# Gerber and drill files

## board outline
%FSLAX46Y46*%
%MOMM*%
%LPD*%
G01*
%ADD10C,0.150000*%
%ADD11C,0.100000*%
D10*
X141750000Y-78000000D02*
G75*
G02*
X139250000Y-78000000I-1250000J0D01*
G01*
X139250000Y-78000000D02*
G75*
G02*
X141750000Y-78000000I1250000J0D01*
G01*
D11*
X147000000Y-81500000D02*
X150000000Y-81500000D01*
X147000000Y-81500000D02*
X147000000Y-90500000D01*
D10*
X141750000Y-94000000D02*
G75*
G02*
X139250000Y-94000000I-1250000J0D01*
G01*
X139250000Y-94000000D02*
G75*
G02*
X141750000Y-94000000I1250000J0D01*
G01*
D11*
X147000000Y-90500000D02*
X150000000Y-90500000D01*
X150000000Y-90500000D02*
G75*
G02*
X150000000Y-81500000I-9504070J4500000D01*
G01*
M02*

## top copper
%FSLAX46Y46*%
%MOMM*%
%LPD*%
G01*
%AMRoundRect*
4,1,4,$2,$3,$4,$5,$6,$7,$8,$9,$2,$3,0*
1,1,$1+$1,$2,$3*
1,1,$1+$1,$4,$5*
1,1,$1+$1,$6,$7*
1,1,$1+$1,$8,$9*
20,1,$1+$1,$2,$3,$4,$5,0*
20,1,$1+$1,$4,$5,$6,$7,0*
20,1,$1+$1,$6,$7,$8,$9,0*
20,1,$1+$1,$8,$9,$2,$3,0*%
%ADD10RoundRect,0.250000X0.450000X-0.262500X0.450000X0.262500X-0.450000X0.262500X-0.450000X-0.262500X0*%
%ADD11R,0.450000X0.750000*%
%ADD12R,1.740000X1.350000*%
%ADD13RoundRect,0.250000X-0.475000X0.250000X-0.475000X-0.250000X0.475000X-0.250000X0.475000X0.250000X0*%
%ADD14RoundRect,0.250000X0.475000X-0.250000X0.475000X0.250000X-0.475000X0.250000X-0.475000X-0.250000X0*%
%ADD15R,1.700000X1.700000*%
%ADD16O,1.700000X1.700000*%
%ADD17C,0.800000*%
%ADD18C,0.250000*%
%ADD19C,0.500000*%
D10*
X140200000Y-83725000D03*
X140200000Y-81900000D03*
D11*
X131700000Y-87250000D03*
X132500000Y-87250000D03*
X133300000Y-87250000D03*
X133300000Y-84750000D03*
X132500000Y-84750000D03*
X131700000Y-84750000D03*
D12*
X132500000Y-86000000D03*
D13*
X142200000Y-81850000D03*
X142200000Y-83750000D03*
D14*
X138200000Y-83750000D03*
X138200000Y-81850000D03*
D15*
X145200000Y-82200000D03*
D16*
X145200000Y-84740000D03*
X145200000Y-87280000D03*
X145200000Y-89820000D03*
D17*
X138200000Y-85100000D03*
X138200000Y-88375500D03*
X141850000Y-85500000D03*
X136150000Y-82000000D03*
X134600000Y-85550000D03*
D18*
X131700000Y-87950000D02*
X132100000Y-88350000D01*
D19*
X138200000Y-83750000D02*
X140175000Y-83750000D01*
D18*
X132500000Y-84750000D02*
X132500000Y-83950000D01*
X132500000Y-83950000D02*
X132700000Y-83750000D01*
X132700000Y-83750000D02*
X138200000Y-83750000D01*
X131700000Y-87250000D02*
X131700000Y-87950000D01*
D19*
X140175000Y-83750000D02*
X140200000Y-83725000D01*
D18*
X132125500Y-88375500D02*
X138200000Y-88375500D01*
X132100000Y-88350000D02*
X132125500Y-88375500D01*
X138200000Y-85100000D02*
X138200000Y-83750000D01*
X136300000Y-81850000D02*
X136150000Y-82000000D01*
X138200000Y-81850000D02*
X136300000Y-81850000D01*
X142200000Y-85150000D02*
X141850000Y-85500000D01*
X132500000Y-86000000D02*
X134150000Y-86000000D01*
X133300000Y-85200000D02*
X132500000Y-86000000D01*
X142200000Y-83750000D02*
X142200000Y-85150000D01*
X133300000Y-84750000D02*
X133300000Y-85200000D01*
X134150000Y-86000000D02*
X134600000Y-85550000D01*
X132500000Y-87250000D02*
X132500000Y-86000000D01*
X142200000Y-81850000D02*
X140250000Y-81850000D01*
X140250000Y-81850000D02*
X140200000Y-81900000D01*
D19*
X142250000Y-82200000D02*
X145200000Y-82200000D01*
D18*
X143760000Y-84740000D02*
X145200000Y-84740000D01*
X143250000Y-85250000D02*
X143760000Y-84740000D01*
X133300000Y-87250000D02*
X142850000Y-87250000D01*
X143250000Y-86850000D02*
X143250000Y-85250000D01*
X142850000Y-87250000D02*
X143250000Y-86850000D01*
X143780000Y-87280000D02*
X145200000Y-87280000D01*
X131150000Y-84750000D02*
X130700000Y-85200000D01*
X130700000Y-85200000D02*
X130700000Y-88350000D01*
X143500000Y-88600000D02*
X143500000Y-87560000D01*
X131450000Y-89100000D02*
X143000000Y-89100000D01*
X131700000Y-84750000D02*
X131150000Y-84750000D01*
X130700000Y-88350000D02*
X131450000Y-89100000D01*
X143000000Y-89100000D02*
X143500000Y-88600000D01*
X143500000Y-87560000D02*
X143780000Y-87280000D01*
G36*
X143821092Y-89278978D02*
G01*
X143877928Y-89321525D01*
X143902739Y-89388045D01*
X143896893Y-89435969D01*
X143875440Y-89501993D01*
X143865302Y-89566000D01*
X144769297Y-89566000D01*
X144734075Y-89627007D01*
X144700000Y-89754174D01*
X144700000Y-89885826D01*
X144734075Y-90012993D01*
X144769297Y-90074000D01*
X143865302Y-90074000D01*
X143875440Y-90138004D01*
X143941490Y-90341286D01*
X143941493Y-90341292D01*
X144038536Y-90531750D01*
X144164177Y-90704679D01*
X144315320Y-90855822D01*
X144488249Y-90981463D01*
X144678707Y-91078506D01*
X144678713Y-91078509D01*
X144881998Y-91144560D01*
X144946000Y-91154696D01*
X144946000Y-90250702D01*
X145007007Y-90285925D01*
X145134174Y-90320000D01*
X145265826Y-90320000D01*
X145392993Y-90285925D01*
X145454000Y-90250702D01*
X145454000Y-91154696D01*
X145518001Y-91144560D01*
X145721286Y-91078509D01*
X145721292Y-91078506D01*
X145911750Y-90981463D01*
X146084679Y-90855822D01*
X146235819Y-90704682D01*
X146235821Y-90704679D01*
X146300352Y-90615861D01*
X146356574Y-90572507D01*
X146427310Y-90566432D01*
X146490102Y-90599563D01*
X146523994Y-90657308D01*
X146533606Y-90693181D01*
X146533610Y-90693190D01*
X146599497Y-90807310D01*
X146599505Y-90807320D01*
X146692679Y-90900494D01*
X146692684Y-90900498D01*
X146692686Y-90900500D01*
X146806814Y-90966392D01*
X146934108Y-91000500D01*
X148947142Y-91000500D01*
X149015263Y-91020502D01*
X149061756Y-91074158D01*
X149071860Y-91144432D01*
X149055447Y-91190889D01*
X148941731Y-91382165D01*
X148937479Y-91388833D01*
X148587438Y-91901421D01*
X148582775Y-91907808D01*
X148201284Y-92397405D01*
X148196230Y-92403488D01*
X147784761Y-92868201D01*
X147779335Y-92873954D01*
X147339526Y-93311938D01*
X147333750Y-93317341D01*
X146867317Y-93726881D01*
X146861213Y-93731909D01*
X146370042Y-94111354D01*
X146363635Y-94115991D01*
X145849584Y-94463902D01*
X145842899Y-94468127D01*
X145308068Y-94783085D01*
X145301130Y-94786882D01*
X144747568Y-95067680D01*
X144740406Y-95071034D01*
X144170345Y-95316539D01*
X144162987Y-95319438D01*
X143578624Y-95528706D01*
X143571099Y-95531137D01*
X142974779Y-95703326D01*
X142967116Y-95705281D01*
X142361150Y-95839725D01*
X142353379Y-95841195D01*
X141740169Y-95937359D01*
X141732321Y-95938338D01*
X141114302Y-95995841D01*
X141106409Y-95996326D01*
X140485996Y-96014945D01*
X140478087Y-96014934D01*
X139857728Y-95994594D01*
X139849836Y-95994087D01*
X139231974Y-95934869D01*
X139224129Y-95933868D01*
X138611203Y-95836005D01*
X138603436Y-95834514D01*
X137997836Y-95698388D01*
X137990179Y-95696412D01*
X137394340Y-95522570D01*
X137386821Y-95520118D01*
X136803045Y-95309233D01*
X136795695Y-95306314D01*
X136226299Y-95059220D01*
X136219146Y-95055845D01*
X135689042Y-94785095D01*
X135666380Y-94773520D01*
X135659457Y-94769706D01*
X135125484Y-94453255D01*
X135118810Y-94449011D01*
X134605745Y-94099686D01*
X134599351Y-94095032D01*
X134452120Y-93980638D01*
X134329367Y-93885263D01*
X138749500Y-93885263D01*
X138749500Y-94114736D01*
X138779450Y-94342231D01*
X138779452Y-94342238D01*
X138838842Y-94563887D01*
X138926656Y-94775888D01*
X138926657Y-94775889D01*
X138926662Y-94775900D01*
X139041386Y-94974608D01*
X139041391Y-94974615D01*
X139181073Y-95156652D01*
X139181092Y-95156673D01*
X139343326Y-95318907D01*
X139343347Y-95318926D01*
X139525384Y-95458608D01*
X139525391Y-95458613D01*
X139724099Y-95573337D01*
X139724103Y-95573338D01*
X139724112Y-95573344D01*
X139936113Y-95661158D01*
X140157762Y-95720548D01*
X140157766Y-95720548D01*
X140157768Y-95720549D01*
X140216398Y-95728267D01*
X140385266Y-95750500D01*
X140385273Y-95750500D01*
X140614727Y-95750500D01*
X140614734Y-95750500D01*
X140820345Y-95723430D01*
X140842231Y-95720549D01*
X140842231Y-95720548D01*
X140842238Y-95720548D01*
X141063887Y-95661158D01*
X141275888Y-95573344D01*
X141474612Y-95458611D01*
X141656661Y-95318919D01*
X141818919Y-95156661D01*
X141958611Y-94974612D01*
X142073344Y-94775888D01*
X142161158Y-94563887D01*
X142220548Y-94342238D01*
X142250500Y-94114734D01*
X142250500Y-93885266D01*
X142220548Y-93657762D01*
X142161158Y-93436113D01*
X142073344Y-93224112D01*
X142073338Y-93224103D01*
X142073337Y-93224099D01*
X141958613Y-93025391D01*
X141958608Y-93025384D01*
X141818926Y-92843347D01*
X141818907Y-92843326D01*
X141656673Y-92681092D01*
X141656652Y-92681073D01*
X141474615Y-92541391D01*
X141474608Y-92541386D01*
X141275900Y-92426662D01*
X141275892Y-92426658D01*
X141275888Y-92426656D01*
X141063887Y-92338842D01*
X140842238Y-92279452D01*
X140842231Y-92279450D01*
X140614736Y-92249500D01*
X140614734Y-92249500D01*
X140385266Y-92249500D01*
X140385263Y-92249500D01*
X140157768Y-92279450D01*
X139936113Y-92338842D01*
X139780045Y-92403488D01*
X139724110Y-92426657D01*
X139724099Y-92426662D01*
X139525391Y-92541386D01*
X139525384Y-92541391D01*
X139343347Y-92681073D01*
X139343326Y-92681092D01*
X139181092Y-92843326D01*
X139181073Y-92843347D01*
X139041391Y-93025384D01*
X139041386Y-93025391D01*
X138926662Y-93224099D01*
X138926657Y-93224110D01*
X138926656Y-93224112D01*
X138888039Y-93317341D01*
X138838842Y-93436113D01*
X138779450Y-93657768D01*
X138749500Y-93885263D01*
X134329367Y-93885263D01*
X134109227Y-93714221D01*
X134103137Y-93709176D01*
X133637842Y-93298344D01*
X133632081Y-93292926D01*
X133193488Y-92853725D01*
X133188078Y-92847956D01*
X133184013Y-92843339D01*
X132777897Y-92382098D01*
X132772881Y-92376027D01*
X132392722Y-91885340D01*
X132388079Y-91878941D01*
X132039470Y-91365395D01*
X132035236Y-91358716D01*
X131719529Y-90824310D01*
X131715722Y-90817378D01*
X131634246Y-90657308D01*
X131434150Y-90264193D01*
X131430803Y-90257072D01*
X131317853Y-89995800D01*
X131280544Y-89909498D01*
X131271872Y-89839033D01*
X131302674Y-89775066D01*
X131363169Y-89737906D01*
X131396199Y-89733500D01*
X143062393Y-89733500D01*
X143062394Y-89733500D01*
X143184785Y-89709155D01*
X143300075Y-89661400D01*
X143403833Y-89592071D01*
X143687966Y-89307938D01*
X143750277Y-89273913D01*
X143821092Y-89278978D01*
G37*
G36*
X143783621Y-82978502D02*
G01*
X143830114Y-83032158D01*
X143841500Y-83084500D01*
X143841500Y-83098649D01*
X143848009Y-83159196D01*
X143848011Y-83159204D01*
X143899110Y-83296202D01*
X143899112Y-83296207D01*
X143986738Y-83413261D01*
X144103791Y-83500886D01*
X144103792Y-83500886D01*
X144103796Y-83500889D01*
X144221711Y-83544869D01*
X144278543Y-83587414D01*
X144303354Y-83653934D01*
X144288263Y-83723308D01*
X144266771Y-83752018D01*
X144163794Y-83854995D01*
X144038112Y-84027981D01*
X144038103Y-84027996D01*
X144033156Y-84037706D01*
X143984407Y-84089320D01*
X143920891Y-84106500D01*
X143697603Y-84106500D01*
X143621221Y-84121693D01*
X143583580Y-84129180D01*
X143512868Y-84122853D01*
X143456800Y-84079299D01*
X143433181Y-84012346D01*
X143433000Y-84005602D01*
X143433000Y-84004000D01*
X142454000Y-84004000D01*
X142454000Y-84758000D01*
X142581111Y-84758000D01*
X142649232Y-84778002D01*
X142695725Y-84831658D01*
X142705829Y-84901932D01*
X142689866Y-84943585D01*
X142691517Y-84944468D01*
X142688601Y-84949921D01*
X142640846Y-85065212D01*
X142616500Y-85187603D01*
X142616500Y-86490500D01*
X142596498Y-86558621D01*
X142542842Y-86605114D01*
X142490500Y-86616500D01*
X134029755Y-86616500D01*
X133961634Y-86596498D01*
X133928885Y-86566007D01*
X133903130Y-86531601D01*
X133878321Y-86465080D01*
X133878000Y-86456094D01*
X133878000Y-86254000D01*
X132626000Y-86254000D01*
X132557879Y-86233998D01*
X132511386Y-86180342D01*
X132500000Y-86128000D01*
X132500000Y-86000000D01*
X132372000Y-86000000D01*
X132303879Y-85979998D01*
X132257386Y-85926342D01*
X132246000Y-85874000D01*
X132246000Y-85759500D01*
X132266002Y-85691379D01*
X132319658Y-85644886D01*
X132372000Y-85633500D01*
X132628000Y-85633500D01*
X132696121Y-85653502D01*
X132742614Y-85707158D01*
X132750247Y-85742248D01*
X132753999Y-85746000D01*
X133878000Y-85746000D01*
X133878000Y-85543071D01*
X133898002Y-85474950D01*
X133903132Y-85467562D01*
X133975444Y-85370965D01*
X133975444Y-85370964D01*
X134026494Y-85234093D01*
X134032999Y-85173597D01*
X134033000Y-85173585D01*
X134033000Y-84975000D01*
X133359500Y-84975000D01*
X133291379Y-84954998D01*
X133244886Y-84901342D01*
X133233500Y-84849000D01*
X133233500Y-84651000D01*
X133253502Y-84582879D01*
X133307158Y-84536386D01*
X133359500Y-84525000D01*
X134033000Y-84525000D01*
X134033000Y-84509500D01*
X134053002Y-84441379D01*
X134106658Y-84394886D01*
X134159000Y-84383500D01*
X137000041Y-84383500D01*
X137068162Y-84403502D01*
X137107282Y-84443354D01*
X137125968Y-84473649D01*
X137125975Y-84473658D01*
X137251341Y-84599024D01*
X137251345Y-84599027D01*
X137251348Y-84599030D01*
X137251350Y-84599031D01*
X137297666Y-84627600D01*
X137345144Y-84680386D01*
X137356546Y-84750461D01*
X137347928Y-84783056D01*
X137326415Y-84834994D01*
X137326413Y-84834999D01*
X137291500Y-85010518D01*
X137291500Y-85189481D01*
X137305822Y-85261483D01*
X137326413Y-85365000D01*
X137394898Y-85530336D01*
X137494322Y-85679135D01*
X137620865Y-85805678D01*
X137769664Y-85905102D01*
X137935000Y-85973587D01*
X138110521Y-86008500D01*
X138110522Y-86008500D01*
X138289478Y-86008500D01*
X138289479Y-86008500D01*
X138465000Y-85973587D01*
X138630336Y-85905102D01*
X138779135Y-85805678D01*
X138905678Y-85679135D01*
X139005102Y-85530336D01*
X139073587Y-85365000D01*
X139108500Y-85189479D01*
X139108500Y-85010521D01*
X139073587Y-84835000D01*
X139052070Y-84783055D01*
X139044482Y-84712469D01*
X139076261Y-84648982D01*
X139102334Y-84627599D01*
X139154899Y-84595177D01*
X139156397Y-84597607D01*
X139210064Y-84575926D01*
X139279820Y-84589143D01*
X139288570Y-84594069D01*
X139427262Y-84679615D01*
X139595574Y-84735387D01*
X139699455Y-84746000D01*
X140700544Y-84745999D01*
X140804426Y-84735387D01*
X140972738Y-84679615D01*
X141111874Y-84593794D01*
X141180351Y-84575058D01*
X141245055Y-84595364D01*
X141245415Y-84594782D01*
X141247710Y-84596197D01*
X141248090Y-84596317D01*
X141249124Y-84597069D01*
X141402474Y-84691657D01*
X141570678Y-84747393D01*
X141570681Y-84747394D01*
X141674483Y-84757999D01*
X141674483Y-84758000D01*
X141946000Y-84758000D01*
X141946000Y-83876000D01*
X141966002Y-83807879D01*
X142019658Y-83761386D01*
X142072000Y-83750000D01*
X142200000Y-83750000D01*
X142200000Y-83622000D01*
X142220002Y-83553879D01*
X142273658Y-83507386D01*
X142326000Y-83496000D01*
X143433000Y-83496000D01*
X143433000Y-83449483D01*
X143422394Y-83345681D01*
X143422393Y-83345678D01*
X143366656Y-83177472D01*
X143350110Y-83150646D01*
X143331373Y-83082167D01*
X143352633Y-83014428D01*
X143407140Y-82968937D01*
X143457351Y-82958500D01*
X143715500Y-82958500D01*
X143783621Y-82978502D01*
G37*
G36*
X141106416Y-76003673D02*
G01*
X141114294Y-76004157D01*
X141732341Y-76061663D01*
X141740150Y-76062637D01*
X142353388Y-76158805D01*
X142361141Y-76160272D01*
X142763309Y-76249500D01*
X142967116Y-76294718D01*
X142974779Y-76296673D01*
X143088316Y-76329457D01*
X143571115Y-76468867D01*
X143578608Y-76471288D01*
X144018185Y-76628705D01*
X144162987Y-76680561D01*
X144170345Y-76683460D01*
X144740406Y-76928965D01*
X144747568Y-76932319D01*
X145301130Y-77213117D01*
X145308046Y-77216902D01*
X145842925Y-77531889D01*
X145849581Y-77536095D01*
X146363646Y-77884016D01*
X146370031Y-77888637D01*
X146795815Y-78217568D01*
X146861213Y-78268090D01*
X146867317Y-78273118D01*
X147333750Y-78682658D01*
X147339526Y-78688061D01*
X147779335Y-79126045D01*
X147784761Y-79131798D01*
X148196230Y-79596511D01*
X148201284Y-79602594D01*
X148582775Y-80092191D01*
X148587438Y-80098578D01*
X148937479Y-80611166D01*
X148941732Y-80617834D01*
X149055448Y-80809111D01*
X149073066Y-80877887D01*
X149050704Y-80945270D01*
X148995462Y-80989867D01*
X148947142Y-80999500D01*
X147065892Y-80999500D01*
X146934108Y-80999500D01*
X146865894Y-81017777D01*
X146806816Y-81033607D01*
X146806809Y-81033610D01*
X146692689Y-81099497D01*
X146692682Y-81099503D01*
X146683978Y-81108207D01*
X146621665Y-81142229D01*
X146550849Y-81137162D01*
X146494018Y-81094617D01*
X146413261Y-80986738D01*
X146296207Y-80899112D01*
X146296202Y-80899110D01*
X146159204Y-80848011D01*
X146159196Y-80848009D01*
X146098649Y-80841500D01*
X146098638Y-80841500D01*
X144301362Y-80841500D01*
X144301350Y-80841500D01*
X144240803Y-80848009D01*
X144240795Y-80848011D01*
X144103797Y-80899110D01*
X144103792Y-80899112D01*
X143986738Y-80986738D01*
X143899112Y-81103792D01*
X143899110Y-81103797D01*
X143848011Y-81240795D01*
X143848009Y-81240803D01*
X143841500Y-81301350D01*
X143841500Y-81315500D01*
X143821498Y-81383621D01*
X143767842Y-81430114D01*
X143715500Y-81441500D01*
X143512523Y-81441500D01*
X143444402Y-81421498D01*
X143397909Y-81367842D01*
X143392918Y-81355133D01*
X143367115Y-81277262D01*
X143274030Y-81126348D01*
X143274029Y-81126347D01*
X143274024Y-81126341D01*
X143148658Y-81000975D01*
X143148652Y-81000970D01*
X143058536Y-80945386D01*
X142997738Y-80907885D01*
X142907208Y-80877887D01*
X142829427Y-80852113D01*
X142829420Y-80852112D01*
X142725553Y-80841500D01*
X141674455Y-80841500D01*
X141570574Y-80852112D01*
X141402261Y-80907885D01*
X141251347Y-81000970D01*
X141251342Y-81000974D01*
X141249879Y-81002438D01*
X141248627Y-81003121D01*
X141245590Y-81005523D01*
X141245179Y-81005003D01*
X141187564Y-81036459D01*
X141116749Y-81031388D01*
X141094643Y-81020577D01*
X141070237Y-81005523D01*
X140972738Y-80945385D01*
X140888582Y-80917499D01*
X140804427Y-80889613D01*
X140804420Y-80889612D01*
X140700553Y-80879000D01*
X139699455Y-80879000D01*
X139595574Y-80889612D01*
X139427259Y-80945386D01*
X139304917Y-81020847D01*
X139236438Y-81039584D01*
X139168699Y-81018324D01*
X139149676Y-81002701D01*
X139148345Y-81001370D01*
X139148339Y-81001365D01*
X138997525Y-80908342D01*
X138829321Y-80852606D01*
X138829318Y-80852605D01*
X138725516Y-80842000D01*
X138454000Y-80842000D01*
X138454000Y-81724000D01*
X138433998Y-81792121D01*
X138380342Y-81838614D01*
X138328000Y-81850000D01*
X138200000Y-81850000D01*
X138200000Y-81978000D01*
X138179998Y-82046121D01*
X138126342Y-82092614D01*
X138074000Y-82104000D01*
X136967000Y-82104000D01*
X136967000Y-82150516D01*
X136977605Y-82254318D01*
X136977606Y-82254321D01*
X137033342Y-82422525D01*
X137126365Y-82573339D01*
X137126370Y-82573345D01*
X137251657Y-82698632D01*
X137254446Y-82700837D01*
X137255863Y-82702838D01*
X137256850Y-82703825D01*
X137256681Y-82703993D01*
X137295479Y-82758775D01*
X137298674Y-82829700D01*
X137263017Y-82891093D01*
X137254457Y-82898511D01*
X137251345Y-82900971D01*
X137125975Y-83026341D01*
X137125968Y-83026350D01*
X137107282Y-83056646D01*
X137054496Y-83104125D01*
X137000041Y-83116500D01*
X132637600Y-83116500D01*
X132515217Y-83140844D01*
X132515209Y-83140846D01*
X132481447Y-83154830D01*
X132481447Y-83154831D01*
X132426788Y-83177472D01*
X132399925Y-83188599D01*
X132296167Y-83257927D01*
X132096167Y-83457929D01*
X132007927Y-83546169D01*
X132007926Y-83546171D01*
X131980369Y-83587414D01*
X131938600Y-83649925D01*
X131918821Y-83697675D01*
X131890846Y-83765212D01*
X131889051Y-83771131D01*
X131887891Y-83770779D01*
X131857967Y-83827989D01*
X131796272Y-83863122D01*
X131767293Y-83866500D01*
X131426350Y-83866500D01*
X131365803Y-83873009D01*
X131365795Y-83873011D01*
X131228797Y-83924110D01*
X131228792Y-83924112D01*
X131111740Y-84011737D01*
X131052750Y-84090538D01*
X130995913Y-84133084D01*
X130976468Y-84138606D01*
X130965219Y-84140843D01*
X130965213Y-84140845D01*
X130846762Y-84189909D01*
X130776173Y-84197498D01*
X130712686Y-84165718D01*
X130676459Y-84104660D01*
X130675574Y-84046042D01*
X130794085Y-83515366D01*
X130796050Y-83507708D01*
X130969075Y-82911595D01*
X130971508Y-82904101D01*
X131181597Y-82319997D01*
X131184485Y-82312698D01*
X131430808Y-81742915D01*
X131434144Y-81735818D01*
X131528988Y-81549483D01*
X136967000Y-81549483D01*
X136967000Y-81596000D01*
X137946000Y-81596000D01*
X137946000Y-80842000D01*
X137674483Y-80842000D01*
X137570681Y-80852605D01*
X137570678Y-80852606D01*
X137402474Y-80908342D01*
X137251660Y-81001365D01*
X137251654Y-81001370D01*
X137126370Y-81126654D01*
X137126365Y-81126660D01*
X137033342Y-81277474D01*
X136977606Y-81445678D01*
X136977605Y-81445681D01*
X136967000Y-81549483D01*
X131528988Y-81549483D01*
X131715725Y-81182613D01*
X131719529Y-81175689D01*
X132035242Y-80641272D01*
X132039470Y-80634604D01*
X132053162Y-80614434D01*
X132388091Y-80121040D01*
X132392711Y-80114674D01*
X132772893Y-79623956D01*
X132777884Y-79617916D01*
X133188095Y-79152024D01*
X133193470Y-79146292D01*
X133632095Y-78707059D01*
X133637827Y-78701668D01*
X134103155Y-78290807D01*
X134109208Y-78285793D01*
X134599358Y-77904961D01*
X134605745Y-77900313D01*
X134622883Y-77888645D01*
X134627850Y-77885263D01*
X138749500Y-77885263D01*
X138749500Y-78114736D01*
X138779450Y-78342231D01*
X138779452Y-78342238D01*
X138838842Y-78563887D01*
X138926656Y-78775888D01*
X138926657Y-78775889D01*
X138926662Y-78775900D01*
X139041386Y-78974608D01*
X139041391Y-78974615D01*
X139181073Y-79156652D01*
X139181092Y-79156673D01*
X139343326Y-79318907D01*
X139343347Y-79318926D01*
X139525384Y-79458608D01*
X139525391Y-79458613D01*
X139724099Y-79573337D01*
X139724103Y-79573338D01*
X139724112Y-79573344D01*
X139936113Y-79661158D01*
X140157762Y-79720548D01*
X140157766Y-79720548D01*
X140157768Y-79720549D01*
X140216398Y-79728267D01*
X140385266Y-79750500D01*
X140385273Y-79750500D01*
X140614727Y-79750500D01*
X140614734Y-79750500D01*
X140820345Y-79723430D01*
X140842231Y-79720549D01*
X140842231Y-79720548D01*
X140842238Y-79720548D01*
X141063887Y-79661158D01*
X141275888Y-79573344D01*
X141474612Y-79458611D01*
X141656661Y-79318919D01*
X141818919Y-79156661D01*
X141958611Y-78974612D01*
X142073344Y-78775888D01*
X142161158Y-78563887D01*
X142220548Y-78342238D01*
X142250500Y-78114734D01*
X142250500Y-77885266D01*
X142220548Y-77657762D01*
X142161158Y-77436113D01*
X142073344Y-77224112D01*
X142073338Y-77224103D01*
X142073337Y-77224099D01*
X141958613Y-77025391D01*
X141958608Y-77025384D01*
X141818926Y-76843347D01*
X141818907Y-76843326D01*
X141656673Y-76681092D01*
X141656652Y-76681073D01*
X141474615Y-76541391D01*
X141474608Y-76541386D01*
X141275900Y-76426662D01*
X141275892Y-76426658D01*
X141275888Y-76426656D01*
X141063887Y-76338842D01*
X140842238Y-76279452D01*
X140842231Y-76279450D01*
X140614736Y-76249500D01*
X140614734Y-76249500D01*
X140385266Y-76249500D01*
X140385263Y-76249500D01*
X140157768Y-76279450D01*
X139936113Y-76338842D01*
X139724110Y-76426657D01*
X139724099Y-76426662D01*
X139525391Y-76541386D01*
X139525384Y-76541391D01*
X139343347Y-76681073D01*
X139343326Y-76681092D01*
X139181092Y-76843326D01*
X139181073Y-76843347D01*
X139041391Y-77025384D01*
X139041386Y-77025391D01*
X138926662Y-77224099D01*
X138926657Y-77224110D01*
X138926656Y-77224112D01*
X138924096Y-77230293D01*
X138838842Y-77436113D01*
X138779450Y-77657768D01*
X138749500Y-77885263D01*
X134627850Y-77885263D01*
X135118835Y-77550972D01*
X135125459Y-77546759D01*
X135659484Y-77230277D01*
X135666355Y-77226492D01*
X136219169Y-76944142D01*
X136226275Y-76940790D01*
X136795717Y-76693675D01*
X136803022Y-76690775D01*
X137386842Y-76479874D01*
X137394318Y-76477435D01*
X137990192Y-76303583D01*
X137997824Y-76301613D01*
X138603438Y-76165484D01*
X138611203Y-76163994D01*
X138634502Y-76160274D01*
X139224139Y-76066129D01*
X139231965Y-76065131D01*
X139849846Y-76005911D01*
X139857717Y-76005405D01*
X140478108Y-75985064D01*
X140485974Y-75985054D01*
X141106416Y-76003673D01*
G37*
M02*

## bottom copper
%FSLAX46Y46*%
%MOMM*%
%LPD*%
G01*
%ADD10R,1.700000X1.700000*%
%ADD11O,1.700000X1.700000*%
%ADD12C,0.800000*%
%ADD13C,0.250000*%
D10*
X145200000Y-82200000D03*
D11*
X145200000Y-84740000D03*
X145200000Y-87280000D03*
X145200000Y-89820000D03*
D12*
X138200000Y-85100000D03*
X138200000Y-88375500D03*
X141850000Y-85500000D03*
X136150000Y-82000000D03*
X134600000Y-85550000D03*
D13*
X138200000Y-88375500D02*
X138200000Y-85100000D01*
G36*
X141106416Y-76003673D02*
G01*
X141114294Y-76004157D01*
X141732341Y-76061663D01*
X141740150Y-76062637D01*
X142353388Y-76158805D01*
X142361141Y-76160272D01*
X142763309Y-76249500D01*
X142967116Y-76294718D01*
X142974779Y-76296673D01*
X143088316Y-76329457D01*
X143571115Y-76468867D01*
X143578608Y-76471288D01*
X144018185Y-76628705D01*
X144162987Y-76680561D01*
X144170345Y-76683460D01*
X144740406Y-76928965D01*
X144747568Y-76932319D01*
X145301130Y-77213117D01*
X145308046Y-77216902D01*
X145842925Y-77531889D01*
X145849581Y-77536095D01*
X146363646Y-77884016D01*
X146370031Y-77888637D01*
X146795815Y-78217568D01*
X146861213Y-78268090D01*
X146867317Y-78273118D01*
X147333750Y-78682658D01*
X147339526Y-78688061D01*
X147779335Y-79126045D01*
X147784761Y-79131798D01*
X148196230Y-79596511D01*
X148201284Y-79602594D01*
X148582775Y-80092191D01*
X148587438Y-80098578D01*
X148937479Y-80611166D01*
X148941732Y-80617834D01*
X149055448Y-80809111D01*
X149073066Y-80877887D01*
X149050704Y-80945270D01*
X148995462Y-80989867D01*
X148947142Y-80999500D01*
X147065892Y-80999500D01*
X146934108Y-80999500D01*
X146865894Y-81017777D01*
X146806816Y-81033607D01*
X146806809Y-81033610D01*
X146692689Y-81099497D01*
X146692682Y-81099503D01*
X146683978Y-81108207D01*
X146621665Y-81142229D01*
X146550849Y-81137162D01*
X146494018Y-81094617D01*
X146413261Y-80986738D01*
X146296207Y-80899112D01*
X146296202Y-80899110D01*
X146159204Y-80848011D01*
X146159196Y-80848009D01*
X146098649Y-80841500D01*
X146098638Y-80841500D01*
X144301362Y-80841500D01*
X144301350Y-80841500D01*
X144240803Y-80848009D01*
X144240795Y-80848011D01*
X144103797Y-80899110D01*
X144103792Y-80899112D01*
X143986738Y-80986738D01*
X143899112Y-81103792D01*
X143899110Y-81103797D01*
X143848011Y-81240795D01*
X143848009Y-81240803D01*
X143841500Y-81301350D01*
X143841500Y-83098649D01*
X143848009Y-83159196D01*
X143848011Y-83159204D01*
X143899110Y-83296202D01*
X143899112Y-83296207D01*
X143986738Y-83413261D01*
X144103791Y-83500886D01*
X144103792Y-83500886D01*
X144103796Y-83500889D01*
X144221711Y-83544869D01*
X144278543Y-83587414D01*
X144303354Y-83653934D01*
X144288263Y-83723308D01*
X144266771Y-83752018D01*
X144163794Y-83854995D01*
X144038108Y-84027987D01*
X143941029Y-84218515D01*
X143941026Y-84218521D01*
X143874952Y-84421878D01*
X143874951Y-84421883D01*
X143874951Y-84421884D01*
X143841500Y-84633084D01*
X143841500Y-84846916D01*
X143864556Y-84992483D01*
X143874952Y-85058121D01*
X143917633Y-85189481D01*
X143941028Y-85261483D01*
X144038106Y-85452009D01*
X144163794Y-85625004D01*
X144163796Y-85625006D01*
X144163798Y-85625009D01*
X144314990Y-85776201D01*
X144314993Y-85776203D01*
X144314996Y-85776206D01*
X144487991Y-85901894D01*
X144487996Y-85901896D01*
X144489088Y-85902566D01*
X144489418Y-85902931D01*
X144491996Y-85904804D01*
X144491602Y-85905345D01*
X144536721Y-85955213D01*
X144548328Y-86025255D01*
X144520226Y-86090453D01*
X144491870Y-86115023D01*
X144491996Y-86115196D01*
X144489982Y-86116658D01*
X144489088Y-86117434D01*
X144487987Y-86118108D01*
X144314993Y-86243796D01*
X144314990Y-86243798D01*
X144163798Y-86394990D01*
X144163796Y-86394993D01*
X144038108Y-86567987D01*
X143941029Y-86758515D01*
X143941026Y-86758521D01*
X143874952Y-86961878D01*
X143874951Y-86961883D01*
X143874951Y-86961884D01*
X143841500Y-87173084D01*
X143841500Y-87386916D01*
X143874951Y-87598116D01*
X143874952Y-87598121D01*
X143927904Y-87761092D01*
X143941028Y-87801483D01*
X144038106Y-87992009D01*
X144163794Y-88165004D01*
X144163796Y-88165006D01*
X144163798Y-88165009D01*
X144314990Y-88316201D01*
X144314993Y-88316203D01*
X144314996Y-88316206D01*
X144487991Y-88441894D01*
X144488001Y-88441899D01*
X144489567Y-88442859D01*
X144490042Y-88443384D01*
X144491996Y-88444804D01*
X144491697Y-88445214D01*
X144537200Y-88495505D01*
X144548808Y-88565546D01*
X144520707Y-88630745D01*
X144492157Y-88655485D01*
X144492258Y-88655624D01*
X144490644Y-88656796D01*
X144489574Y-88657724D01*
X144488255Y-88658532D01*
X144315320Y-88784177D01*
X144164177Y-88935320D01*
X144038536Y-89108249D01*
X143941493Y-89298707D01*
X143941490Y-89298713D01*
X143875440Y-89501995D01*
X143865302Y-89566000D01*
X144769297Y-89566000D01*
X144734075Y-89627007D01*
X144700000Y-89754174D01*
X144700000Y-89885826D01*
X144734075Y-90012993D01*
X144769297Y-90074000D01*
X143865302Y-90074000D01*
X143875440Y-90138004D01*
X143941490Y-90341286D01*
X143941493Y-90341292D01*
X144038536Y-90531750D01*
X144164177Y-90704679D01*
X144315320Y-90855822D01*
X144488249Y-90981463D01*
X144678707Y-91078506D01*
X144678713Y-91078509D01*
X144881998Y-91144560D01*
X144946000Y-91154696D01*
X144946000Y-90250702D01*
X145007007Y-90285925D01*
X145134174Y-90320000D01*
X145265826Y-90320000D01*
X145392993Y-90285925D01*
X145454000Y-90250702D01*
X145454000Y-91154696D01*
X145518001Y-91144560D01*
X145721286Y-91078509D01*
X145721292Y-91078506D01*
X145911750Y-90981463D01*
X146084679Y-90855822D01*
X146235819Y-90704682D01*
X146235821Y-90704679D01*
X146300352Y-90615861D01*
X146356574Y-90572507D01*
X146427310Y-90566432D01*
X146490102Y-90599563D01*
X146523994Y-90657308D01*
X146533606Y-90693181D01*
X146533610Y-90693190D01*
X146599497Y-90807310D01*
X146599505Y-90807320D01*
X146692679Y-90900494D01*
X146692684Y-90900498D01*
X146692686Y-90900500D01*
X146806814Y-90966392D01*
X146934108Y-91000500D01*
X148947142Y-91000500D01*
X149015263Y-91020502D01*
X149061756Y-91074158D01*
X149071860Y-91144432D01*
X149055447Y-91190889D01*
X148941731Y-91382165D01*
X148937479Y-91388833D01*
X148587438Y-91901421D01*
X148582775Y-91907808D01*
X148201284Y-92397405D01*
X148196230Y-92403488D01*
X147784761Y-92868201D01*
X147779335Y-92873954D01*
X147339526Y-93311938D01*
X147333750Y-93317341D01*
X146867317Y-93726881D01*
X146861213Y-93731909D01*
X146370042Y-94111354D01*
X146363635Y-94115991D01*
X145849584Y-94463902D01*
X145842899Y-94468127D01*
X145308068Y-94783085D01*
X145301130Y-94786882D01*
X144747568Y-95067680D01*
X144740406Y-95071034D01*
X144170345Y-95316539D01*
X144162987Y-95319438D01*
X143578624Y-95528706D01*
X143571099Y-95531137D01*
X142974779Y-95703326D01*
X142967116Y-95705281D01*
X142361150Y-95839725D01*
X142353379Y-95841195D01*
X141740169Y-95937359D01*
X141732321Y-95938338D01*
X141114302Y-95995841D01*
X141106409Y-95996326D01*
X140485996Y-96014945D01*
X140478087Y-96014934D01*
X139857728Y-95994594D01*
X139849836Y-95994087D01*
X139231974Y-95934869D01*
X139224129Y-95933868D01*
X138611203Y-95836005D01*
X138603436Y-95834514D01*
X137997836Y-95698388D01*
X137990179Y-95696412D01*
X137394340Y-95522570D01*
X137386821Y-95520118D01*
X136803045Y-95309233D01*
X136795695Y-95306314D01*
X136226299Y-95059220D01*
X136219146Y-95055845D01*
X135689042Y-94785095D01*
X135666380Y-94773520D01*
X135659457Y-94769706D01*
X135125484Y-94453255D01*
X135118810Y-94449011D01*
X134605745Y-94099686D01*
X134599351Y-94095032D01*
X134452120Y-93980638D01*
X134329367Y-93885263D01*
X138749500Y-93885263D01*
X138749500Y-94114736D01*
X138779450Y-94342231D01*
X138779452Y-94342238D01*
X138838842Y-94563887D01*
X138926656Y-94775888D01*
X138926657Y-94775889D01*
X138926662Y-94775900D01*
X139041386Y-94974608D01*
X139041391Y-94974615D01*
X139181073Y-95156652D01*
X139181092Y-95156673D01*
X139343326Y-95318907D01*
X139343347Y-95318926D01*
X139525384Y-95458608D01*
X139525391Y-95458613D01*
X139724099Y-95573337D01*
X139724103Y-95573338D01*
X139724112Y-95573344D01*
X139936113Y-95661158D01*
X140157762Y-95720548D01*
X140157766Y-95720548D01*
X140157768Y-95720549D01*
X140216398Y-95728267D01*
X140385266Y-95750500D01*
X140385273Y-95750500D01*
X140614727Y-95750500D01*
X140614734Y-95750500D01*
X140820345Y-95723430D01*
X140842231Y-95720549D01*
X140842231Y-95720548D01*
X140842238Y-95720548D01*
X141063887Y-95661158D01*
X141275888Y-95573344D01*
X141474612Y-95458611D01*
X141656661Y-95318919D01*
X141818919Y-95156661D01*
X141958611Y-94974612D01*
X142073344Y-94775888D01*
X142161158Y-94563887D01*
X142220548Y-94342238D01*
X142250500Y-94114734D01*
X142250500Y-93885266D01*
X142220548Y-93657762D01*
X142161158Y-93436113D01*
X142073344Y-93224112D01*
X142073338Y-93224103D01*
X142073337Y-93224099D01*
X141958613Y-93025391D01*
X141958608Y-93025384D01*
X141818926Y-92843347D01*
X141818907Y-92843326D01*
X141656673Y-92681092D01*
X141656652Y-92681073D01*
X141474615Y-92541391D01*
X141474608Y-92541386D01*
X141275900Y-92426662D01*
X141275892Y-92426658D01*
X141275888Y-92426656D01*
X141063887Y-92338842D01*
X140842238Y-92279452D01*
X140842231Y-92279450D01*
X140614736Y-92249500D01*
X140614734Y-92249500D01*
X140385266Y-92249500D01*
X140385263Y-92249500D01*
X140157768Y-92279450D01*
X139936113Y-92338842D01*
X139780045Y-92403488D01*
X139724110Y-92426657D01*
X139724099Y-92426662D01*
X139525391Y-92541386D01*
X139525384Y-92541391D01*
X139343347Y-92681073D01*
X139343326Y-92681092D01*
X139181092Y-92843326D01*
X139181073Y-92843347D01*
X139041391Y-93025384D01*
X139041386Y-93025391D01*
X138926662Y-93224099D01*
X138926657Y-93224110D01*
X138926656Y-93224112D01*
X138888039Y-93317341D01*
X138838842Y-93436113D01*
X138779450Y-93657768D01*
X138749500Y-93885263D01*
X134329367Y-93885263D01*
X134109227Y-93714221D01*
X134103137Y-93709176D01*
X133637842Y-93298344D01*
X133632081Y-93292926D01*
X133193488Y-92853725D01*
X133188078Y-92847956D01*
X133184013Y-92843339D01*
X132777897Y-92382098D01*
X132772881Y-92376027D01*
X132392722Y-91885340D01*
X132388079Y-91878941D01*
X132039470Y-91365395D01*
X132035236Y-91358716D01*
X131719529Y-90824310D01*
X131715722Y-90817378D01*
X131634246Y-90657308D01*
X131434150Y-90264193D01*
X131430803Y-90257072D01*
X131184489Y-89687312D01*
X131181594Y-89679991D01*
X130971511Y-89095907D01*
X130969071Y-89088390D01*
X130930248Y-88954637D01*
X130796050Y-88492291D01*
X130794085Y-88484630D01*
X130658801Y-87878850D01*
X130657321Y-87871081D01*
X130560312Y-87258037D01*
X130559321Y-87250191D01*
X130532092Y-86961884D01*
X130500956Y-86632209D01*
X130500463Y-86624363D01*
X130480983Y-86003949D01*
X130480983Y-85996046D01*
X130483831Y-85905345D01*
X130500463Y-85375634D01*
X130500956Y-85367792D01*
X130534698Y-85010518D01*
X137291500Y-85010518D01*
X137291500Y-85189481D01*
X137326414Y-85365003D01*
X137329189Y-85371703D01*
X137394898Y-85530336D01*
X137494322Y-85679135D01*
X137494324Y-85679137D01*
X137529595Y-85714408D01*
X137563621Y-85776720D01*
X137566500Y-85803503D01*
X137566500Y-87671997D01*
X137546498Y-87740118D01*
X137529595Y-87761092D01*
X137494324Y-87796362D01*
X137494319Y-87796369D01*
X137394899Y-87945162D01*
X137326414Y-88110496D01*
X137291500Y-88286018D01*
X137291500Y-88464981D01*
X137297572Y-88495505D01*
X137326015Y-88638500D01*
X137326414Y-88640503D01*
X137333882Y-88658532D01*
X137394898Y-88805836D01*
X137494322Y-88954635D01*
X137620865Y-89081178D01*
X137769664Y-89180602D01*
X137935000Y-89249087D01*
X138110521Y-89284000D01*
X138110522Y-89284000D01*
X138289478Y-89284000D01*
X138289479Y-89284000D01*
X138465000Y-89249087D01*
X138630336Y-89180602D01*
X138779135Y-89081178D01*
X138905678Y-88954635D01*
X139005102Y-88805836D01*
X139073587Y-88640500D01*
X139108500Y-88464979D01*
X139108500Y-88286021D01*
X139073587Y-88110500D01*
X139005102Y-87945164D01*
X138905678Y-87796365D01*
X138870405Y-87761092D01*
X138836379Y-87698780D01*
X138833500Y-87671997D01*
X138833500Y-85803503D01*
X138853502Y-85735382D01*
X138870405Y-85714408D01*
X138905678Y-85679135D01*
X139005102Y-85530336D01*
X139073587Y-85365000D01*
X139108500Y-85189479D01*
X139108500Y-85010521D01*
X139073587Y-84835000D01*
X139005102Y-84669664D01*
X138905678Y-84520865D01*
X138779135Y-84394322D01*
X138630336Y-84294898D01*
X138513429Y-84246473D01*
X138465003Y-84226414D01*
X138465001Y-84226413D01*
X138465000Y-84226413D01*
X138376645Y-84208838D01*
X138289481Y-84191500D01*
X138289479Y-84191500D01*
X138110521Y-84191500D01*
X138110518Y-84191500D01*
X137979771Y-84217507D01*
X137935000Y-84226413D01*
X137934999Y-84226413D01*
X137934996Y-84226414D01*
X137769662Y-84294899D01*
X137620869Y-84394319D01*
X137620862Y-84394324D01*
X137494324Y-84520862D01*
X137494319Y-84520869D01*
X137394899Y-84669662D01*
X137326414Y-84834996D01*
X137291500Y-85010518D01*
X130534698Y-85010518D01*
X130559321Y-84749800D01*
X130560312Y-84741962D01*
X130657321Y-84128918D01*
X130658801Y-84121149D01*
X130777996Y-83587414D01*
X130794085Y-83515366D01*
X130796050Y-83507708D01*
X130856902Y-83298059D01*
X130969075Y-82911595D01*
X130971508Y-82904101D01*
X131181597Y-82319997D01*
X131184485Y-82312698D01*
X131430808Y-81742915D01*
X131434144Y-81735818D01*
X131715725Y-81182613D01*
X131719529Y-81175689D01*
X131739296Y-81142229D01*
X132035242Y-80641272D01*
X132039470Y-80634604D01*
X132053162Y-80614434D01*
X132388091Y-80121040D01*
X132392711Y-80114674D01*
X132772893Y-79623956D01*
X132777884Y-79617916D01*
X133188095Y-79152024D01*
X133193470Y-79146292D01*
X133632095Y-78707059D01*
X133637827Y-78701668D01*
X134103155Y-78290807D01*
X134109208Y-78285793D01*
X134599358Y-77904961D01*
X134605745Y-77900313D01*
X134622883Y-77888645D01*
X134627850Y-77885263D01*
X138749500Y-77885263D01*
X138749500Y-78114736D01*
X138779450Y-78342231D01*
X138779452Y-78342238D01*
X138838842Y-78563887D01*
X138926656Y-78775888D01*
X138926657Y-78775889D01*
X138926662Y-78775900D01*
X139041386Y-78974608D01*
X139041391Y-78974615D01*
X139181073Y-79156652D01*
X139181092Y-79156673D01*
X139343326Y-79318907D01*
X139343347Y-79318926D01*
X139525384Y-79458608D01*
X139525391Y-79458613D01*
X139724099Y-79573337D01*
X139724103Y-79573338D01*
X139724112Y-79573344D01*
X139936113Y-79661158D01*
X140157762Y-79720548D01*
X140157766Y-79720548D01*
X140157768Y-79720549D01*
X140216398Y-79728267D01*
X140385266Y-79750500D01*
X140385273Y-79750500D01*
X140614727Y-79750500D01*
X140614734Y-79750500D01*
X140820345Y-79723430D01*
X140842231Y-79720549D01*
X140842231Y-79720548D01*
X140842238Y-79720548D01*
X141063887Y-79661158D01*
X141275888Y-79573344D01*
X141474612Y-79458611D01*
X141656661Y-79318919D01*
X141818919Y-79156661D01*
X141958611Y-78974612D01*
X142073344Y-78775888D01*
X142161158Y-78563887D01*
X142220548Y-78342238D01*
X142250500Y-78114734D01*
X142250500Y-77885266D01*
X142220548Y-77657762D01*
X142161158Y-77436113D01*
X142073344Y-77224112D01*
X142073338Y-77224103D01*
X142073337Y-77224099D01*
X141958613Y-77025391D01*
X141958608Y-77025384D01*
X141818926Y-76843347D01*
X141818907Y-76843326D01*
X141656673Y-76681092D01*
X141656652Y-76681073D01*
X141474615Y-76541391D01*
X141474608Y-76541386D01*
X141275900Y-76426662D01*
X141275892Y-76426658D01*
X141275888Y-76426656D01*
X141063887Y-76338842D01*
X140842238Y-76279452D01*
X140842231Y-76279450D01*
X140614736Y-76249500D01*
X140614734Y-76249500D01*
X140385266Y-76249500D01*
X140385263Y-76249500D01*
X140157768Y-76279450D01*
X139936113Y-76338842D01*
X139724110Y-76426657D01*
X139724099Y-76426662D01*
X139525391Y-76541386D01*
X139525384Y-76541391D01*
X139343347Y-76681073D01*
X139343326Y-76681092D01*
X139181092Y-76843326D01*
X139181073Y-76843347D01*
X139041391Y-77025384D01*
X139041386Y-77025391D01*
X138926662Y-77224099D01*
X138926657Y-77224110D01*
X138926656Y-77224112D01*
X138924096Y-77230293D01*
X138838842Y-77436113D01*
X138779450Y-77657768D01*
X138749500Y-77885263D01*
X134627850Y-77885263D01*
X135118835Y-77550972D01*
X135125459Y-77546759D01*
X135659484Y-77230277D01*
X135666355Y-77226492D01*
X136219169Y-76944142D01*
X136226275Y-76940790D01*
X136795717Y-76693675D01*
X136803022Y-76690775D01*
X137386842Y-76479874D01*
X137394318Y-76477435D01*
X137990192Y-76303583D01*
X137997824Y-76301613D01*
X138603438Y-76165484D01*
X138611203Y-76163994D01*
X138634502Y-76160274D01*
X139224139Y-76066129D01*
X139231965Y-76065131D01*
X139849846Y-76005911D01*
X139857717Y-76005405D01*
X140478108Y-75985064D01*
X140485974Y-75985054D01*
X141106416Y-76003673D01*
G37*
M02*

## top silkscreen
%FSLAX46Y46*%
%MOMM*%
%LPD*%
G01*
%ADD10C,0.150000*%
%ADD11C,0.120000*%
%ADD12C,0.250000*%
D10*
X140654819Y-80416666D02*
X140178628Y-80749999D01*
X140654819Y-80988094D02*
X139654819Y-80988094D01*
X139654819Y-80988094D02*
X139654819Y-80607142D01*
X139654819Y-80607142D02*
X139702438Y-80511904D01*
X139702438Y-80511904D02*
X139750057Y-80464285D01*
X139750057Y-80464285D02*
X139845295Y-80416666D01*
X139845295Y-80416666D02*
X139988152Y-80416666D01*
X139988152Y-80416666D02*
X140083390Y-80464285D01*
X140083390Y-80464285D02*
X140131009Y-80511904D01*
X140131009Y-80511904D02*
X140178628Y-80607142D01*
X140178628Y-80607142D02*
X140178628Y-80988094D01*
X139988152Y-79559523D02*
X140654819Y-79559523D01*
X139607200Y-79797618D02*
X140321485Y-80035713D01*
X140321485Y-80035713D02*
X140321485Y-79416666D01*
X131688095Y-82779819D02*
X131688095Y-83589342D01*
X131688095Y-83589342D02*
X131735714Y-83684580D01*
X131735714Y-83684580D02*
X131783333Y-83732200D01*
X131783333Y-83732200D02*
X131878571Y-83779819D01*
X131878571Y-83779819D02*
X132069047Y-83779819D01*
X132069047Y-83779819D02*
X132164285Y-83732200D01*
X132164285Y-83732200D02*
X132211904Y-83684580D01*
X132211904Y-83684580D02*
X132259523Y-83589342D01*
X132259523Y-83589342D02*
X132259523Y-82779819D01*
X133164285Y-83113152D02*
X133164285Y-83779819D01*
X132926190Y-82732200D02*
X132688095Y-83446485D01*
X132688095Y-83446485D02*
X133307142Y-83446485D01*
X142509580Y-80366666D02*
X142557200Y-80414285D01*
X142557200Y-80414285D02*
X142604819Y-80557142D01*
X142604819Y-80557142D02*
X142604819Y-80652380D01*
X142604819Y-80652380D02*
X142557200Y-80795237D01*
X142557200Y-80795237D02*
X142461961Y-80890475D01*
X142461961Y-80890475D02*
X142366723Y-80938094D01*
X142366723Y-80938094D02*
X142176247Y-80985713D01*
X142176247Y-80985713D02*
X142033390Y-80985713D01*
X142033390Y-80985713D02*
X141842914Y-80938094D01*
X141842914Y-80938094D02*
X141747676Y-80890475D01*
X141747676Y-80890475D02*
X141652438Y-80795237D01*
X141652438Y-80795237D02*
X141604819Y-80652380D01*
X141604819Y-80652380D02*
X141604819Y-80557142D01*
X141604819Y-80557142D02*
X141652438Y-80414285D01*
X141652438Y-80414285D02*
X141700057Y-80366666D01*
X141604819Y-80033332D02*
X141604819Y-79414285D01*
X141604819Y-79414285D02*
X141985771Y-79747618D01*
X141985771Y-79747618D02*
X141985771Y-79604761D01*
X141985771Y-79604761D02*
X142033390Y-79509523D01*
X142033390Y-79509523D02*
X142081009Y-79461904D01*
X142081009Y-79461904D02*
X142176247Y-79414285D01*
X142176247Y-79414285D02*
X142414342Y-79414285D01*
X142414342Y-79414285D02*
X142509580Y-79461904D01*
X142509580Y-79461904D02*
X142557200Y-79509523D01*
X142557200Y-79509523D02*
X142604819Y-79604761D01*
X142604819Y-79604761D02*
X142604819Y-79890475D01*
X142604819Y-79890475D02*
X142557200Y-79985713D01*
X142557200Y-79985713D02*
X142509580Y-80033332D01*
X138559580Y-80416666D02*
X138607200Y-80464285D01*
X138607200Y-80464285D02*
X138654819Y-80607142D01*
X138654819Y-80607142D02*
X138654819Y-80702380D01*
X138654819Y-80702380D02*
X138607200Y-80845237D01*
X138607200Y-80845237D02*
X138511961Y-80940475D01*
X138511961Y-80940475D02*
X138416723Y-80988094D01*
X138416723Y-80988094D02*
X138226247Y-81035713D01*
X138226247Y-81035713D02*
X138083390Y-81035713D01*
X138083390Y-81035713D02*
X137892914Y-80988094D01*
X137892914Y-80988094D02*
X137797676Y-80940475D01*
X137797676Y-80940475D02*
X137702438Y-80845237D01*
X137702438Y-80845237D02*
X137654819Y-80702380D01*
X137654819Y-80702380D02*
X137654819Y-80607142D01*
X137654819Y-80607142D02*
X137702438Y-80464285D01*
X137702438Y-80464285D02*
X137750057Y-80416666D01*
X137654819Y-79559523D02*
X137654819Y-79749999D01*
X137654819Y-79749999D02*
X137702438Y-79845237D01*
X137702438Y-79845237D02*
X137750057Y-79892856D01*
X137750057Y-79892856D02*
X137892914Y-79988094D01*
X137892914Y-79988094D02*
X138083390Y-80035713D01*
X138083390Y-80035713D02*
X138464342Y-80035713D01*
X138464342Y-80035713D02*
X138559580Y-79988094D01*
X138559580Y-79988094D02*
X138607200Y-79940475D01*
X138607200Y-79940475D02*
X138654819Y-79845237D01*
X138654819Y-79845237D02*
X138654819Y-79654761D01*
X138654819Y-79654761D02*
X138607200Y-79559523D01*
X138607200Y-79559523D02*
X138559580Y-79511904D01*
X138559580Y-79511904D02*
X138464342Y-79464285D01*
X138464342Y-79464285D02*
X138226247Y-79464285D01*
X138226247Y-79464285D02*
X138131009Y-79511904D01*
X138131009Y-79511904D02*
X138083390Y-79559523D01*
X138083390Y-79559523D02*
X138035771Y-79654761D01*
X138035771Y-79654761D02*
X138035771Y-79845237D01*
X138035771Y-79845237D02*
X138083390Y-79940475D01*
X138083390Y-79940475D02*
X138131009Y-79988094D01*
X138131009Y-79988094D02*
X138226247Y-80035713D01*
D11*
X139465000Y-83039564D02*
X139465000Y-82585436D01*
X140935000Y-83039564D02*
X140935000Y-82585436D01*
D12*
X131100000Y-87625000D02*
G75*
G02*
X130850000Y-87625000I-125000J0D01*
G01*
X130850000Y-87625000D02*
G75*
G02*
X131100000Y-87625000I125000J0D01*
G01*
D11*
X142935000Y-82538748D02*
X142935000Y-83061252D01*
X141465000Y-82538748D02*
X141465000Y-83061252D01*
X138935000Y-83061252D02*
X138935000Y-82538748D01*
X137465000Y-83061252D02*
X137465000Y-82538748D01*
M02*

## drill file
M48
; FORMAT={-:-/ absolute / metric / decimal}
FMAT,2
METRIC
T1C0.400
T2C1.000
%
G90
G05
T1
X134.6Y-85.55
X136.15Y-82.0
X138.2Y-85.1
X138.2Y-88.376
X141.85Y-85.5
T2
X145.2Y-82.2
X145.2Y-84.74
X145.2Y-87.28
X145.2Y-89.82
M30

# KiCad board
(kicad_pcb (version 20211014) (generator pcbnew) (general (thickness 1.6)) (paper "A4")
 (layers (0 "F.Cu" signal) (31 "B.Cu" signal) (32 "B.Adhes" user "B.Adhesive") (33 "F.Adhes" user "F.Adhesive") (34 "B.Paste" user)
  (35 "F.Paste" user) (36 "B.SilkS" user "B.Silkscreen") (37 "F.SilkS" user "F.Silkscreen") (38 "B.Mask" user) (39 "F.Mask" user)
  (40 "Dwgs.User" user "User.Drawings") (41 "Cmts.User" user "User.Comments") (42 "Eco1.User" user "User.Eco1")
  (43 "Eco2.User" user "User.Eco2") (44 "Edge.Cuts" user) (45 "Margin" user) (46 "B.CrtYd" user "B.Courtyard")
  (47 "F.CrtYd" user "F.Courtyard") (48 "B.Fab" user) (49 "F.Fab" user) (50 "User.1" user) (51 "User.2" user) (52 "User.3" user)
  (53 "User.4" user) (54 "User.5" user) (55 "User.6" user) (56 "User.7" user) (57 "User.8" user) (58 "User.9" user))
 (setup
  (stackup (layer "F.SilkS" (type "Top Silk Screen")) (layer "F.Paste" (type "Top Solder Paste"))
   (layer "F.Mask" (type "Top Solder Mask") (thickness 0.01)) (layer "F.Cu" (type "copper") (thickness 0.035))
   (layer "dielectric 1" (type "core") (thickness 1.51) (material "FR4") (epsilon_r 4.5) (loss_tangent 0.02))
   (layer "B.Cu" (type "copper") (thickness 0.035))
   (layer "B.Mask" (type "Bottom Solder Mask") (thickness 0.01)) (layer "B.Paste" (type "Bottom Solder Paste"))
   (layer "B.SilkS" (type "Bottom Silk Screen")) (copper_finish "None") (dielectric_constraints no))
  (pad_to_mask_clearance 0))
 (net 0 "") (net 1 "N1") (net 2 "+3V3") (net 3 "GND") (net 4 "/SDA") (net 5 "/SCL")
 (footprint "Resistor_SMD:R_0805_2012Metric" (layer "F.Cu") (at 140.2 82.8125 90)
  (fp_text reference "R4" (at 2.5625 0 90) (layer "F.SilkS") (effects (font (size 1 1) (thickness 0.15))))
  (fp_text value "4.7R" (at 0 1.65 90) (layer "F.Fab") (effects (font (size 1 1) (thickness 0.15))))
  (fp_line (start -0.227064 -0.735) (end 0.227064 -0.735) (layer "F.SilkS") (width 0.12))
  (fp_line (start -0.227064 0.735) (end 0.227064 0.735) (layer "F.SilkS") (width 0.12))
  (pad "1" smd roundrect locked (at -0.9125 0 90) (size 1.025 1.4) (layers "F.Cu" "F.Paste" "F.Mask") (roundrect_rratio 0.243902439)
   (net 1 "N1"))
  (pad "2" smd roundrect locked (at 0.9125 0 90) (size 1.025 1.4) (layers "F.Cu" "F.Paste" "F.Mask") (roundrect_rratio 0.243902439)
   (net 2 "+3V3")))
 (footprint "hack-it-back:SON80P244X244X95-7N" (layer "F.Cu") (at 132.5 86 90)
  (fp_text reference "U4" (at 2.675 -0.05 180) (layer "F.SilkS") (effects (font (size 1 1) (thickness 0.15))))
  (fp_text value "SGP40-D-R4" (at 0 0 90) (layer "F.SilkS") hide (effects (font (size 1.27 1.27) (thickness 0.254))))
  (fp_circle (center -1.625 -1.525) (end -1.625 -1.4) (layer "F.SilkS") (width 0.25) (fill none))
  (pad "1" smd rect (at -1.25 -0.8 180) (size 0.45 0.75) (layers "F.Cu" "F.Paste" "F.Mask") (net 1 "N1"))
  (pad "2" smd rect (at -1.25 0 180) (size 0.45 0.75) (layers "F.Cu" "F.Paste" "F.Mask") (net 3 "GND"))
  (pad "3" smd rect (at -1.25 0.8 180) (size 0.45 0.75) (layers "F.Cu" "F.Paste" "F.Mask") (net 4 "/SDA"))
  (pad "4" smd rect (at 1.25 0.8 180) (size 0.45 0.75) (layers "F.Cu" "F.Paste" "F.Mask") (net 3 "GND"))
  (pad "5" smd rect (at 1.25 0 180) (size 0.45 0.75) (layers "F.Cu" "F.Paste" "F.Mask") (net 1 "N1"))
  (pad "6" smd rect (at 1.25 -0.8 180) (size 0.45 0.75) (layers "F.Cu" "F.Paste" "F.Mask") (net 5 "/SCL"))
  (pad "7" smd rect (at 0 0 90) (size 1.35 1.74) (layers "F.Cu" "F.Paste" "F.Mask") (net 3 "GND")))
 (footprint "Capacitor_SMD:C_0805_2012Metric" (layer "F.Cu") (at 142.2 82.8 -90)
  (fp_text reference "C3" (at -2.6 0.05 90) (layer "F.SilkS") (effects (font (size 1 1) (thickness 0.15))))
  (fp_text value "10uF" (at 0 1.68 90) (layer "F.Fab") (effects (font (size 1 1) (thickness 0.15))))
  (fp_line (start -0.261252 -0.735) (end 0.261252 -0.735) (layer "F.SilkS") (width 0.12))
  (fp_line (start -0.261252 0.735) (end 0.261252 0.735) (layer "F.SilkS") (width 0.12))
  (pad "1" smd roundrect locked (at -0.95 0 270) (size 1 1.45) (layers "F.Cu" "F.Paste" "F.Mask") (roundrect_rratio 0.25) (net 2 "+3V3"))
  (pad "2" smd roundrect locked (at 0.95 0 270) (size 1 1.45) (layers "F.Cu" "F.Paste" "F.Mask") (roundrect_rratio 0.25) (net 3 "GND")))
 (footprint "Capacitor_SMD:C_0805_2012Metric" (layer "F.Cu") (at 138.2 82.8 90)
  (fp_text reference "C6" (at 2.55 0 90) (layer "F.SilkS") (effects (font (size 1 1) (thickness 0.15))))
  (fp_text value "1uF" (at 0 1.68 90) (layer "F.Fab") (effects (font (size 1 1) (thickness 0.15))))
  (fp_line (start -0.261252 0.735) (end 0.261252 0.735) (layer "F.SilkS") (width 0.12))
  (fp_line (start -0.261252 -0.735) (end 0.261252 -0.735) (layer "F.SilkS") (width 0.12))
  (pad "1" smd roundrect locked (at -0.95 0 90) (size 1 1.45) (layers "F.Cu" "F.Paste" "F.Mask") (roundrect_rratio 0.25) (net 1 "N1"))
  (pad "2" smd roundrect locked (at 0.95 0 90) (size 1 1.45) (layers "F.Cu" "F.Paste" "F.Mask") (roundrect_rratio 0.25) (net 3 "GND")))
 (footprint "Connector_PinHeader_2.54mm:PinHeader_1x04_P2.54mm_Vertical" (layer "B.Cu") (at 145.2 82.2 180)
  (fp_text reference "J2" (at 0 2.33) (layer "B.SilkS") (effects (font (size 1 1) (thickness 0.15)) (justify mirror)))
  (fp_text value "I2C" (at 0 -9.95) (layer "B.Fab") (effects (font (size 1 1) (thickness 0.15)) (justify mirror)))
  (pad "1" thru_hole rect locked (at 0 0 180) (size 1.7 1.7) (drill 1) (layers *.Cu *.Mask) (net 2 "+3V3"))
  (pad "2" thru_hole oval locked (at 0 -2.54 180) (size 1.7 1.7) (drill 1) (layers *.Cu *.Mask) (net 4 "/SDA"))
  (pad "3" thru_hole oval locked (at 0 -5.08 180) (size 1.7 1.7) (drill 1) (layers *.Cu *.Mask) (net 5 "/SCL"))
  (pad "4" thru_hole oval locked (at 0 -7.62 180) (size 1.7 1.7) (drill 1) (layers *.Cu *.Mask) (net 3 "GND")))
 (gr_circle (center 140.5 78) (end 141.75 78) (layer "Edge.Cuts") (width 0.15) (fill none))
 (gr_line (start 147 81.5) (end 150 81.5) (layer "Edge.Cuts") (width 0.1))
 (gr_line (start 147 81.5) (end 147 90.5) (layer "Edge.Cuts") (width 0.1))
 (gr_circle (center 140.5 94) (end 141.75 94) (layer "Edge.Cuts") (width 0.15) (fill none))
 (gr_line (start 147 90.5) (end 150 90.5) (layer "Edge.Cuts") (width 0.1))
 (gr_arc (start 150 90.5) (mid 129.980359 86) (end 150 81.5) (layer "Edge.Cuts") (width 0.1))
 (segment (start 131.7 87.95) (end 132.1 88.35) (width 0.25) (layer "F.Cu") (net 1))
 (segment (start 138.2 83.75) (end 140.175 83.75) (width 0.5) (layer "F.Cu") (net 1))
 (segment (start 132.5 84.75) (end 132.5 83.95) (width 0.25) (layer "F.Cu") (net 1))
 (segment (start 132.5 83.95) (end 132.7 83.75) (width 0.25) (layer "F.Cu") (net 1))
 (segment (start 132.7 83.75) (end 138.2 83.75) (width 0.25) (layer "F.Cu") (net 1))
 (segment (start 131.7 87.25) (end 131.7 87.95) (width 0.25) (layer "F.Cu") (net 1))
 (segment (start 140.175 83.75) (end 140.2 83.725) (width 0.5) (layer "F.Cu") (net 1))
 (segment (start 132.1255 88.3755) (end 138.2 88.3755) (width 0.25) (layer "F.Cu") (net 1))
 (segment (start 132.1 88.35) (end 132.1255 88.3755) (width 0.25) (layer "F.Cu") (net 1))
 (segment (start 138.2 85.1) (end 138.2 83.75) (width 0.25) (layer "F.Cu") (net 1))
 (via (at 138.2 85.1) (size 0.8) (drill 0.4) (layers "F.Cu" "B.Cu") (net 1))
 (via (at 138.2 88.3755) (size 0.8) (drill 0.4) (layers "F.Cu" "B.Cu") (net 1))
 (segment (start 138.2 88.3755) (end 138.2 85.1) (width 0.25) (layer "B.Cu") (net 1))
 (segment (start 136.3 81.85) (end 136.15 82) (width 0.25) (layer "F.Cu") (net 3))
 (segment (start 138.2 81.85) (end 136.3 81.85) (width 0.25) (layer "F.Cu") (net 3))
 (segment (start 142.2 85.15) (end 141.85 85.5) (width 0.25) (layer "F.Cu") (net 3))
 (segment (start 132.5 86) (end 134.15 86) (width 0.25) (layer "F.Cu") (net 3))
 (segment (start 133.3 85.2) (end 132.5 86) (width 0.25) (layer "F.Cu") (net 3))
 (segment (start 142.2 83.75) (end 142.2 85.15) (width 0.25) (layer "F.Cu") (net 3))
 (segment (start 133.3 84.75) (end 133.3 85.2) (width 0.25) (layer "F.Cu") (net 3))
 (segment (start 134.15 86) (end 134.6 85.55) (width 0.25) (layer "F.Cu") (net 3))
 (segment (start 132.5 87.25) (end 132.5 86) (width 0.25) (layer "F.Cu") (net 3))
 (via (at 141.85 85.5) (size 0.8) (drill 0.4) (layers "F.Cu" "B.Cu") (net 3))
 (via (at 136.15 82) (size 0.8) (drill 0.4) (layers "F.Cu" "B.Cu") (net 3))
 (via (at 134.6 85.55) (size 0.8) (drill 0.4) (layers "F.Cu" "B.Cu") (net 3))
 (segment (start 142.2 81.85) (end 140.25 81.85) (width 0.25) (layer "F.Cu") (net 2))
 (segment (start 140.25 81.85) (end 140.2 81.9) (width 0.25) (layer "F.Cu") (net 2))
 (segment (start 142.25 82.2) (end 145.2 82.2) (width 0.5) (layer "F.Cu") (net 2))
 (segment (start 143.76 84.74) (end 145.2 84.74) (width 0.25) (layer "F.Cu") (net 4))
 (segment (start 143.25 85.25) (end 143.76 84.74) (width 0.25) (layer "F.Cu") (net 4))
 (segment (start 133.3 87.25) (end 142.85 87.25) (width 0.25) (layer "F.Cu") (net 4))
 (segment (start 143.25 86.85) (end 143.25 85.25) (width 0.25) (layer "F.Cu") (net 4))
 (segment (start 142.85 87.25) (end 143.25 86.85) (width 0.25) (layer "F.Cu") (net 4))
 (segment (start 143.78 87.28) (end 145.2 87.28) (width 0.25) (layer "F.Cu") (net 5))
 (segment (start 131.15 84.75) (end 130.7 85.2) (width 0.25) (layer "F.Cu") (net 5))
 (segment (start 130.7 85.2) (end 130.7 88.35) (width 0.25) (layer "F.Cu") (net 5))
 (segment (start 143.5 88.6) (end 143.5 87.56) (width 0.25) (layer "F.Cu") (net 5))
 (segment (start 131.45 89.1) (end 143 89.1) (width 0.25) (layer "F.Cu") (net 5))
 (segment (start 131.7 84.75) (end 131.15 84.75) (width 0.25) (layer "F.Cu") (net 5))
 (segment (start 130.7 88.35) (end 131.45 89.1) (width 0.25) (layer "F.Cu") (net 5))
 (segment (start 143 89.1) (end 143.5 88.6) (width 0.25) (layer "F.Cu") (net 5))
 (segment (start 143.5 87.56) (end 143.78 87.28) (width 0.25) (layer "F.Cu") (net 5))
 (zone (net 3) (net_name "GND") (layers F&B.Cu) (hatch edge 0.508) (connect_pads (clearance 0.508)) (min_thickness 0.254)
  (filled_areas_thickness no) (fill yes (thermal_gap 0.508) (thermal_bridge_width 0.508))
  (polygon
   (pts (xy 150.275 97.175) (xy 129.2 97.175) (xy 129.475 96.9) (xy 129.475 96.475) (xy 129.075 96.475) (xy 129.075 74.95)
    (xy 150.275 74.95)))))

